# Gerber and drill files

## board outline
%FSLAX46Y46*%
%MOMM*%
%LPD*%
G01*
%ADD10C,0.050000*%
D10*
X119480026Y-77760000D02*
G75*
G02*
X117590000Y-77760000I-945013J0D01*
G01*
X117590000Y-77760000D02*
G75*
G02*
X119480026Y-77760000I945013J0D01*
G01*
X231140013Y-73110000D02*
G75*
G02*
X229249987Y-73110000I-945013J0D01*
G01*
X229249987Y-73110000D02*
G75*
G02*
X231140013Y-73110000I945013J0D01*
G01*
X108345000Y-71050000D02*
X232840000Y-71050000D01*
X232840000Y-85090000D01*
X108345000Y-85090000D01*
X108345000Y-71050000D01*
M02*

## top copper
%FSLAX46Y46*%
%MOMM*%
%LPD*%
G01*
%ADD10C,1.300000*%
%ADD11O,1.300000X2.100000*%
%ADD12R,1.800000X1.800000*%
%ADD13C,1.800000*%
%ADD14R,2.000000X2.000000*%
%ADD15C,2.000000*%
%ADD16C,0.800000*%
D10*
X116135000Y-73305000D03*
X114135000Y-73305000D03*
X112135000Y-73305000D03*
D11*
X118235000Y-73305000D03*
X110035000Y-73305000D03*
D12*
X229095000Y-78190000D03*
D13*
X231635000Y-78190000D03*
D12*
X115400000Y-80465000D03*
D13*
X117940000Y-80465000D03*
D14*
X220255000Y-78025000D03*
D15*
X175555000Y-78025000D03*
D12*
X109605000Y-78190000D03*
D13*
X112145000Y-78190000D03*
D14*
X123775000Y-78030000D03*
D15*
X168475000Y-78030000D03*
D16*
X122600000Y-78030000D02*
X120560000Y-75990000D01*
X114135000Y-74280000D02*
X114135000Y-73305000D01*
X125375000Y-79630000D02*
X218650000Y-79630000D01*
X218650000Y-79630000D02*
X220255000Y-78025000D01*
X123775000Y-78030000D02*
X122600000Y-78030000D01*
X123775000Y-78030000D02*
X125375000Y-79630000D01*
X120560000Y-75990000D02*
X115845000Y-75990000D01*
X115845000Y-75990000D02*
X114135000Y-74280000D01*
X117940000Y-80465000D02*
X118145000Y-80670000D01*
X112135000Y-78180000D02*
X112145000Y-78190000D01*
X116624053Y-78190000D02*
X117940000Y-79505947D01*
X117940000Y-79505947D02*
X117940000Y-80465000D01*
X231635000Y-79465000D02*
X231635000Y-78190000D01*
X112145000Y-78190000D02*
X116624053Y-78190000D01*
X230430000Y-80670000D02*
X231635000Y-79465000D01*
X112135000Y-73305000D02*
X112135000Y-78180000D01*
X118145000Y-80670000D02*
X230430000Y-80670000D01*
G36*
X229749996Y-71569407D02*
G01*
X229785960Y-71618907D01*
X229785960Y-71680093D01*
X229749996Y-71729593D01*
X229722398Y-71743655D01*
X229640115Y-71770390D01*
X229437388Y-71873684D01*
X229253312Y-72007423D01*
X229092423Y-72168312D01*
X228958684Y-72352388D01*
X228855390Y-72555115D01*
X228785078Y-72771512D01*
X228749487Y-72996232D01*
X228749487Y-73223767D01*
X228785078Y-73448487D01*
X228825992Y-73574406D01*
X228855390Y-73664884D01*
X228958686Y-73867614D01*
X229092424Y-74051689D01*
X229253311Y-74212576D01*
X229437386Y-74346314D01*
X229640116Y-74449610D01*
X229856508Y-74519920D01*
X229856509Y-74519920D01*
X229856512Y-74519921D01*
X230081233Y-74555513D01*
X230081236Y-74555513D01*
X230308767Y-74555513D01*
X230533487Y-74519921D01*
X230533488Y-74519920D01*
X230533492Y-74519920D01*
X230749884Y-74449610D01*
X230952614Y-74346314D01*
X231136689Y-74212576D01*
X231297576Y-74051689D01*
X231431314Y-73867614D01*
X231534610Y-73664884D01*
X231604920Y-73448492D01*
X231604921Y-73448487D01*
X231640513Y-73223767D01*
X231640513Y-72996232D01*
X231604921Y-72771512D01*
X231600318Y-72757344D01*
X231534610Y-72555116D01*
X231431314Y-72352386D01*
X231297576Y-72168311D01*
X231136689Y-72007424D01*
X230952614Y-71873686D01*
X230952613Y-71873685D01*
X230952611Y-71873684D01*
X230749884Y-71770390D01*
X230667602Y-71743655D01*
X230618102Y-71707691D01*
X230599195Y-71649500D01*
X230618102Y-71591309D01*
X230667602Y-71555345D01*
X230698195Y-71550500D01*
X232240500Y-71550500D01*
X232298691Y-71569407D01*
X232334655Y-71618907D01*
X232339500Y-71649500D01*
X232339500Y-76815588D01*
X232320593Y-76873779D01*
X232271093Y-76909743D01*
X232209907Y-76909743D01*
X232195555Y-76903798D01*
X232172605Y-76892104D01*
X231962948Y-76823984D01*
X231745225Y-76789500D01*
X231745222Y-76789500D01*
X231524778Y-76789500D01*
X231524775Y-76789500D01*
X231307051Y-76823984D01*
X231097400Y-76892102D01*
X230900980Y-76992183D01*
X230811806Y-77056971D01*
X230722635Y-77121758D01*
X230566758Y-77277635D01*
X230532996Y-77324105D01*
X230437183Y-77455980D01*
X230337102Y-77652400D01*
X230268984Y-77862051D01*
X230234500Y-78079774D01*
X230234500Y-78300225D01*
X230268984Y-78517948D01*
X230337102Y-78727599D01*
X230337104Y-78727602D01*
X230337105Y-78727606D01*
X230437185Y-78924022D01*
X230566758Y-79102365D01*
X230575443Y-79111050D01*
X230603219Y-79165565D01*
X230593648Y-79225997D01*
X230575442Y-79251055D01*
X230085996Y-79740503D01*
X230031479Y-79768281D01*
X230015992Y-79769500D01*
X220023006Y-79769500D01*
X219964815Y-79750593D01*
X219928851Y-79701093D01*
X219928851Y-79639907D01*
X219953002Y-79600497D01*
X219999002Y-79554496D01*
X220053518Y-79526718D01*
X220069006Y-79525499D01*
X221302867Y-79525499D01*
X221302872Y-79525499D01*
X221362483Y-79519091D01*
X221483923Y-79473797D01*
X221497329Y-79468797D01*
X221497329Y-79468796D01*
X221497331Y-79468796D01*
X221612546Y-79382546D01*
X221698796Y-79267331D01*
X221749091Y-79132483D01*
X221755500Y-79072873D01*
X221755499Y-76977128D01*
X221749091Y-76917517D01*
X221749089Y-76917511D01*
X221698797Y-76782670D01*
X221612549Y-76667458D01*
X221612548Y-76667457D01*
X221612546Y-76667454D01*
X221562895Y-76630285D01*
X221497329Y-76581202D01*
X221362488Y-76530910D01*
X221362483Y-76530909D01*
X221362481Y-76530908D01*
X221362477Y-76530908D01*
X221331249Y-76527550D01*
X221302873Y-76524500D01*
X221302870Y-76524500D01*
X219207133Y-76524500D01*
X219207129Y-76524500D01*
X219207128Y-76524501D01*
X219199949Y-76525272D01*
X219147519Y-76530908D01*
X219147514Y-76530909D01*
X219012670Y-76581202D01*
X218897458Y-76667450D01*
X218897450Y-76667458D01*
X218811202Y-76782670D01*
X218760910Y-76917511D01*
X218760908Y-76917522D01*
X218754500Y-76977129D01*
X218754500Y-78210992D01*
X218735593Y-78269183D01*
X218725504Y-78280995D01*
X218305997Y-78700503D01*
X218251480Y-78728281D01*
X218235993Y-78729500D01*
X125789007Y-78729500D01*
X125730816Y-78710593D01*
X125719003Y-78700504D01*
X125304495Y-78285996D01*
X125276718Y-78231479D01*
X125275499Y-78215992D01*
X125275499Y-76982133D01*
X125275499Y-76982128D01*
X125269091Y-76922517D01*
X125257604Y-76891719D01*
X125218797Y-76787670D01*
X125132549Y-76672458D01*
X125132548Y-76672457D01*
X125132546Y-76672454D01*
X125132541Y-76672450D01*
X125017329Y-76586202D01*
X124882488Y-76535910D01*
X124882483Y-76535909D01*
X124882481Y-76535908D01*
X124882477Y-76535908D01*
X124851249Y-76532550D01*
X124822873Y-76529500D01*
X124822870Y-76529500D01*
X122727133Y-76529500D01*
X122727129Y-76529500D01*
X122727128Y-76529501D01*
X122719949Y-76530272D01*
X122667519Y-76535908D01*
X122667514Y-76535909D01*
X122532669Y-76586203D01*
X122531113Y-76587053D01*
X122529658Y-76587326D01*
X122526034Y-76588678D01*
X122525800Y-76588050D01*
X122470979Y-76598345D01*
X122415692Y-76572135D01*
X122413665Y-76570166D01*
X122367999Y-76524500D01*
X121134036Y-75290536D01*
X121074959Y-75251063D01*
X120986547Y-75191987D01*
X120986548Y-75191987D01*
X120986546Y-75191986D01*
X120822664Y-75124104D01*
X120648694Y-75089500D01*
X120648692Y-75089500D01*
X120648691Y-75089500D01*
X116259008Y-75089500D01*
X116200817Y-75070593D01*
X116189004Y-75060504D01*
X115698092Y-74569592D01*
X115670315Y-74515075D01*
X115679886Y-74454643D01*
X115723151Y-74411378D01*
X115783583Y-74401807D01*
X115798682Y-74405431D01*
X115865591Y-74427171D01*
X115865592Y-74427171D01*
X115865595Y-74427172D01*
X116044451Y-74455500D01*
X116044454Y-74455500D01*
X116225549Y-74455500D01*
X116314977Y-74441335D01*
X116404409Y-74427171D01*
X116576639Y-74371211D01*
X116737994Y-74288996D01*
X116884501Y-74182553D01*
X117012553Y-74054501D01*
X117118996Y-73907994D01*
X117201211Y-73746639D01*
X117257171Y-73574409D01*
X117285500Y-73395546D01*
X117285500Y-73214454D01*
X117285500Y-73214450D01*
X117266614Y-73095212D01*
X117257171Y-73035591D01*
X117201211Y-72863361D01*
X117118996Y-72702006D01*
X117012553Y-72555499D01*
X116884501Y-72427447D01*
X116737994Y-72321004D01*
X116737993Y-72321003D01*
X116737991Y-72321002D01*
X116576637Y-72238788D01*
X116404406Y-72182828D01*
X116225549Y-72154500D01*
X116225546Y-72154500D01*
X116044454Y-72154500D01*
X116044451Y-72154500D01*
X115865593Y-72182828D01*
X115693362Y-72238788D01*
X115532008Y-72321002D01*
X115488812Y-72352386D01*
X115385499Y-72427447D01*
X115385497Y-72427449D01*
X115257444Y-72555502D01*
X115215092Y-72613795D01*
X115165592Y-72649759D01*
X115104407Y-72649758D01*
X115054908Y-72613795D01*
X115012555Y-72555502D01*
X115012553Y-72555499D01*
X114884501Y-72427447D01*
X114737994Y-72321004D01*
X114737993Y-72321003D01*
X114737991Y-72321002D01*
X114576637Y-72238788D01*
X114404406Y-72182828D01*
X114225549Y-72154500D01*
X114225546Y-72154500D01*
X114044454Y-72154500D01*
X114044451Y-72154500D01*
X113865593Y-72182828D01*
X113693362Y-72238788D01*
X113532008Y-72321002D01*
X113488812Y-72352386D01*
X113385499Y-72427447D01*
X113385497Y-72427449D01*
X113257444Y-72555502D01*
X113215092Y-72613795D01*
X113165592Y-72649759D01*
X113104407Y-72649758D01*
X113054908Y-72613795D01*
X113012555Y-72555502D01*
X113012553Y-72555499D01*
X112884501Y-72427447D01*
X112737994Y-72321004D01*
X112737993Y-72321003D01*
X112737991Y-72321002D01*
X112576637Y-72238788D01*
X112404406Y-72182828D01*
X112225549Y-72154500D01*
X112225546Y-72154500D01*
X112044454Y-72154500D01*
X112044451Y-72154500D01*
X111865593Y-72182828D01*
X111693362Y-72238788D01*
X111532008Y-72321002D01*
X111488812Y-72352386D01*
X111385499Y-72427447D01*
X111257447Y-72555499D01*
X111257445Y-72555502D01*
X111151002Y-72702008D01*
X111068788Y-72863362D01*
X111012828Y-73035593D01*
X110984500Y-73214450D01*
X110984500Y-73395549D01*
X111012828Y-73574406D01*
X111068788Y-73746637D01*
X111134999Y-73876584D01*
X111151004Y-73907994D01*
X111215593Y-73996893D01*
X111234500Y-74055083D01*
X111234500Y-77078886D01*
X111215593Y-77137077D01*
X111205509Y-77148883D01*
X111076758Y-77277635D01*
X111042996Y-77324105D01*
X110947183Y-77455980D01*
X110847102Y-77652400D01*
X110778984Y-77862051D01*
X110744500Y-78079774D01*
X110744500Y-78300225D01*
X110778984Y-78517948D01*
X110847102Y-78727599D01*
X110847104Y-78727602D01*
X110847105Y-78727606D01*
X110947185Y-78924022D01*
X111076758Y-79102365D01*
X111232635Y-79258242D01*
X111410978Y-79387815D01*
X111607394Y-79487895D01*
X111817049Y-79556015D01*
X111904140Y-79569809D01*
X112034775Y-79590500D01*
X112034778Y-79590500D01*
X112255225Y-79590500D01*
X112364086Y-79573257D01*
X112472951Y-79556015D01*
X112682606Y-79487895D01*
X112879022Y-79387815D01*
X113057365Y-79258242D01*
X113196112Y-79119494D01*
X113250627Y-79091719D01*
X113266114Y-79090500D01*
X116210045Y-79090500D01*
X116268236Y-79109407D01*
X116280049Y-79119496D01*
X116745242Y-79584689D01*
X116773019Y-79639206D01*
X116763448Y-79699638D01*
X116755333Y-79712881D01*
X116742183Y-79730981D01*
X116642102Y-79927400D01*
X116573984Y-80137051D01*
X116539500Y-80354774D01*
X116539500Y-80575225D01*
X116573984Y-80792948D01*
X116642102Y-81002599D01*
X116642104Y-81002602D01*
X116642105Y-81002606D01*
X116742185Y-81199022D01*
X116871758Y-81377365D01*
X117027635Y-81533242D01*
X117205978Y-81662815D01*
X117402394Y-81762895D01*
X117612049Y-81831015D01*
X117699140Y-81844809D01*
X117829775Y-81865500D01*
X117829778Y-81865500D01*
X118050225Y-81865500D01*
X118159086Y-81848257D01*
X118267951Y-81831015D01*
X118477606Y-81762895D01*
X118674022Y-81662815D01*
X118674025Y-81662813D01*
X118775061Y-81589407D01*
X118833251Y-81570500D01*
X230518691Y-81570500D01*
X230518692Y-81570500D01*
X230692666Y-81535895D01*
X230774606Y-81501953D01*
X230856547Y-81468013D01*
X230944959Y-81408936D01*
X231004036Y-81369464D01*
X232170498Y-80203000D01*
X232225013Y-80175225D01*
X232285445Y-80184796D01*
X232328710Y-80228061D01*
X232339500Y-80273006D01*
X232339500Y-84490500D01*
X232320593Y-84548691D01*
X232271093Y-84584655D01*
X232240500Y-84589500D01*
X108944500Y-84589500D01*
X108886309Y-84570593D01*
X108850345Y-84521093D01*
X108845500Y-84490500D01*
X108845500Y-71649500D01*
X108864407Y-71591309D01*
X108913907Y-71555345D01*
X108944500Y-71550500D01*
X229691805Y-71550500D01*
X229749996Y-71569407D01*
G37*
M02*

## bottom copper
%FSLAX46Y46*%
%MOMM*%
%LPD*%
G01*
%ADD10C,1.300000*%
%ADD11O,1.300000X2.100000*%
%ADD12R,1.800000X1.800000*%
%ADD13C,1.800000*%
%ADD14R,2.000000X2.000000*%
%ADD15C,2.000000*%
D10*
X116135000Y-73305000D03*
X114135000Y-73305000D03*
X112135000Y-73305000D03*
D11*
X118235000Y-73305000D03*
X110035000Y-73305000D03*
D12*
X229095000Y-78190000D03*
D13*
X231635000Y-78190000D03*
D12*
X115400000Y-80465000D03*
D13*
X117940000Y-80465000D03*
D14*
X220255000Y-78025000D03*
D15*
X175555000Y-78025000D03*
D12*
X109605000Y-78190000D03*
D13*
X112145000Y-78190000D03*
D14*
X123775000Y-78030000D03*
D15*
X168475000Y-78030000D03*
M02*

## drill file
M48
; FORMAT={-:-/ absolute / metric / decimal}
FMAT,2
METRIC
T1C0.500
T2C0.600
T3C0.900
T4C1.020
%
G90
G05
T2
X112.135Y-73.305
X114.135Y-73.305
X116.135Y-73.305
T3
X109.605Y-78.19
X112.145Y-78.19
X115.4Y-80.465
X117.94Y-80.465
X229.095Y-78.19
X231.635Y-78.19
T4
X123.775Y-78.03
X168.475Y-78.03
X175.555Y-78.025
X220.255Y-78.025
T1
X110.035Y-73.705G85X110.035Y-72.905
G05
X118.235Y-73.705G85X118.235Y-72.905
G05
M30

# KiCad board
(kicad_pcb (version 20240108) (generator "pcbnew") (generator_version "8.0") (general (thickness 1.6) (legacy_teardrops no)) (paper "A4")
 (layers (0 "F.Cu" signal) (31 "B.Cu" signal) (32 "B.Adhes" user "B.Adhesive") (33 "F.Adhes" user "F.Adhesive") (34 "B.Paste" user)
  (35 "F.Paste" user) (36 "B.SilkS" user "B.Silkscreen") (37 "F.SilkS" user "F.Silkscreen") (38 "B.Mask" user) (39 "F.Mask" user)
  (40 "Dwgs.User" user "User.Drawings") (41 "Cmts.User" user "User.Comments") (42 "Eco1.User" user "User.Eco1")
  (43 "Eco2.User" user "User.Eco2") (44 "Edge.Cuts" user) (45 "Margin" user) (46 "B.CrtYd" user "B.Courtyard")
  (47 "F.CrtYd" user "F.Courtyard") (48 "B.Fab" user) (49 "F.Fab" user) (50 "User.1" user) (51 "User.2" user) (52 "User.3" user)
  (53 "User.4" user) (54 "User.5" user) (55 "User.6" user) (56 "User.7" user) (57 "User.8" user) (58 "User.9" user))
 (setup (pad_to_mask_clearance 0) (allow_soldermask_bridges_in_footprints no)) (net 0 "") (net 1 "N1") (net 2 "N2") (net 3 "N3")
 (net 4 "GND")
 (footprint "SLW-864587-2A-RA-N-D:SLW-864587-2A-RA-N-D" (layer "F.Cu") (at 114.135 73.305 180)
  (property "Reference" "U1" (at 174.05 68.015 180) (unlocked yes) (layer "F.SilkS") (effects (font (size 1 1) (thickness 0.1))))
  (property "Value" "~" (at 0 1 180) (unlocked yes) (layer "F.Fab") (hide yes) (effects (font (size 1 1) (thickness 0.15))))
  (pad "1" thru_hole circle (at -2 0 180) (size 1.3 1.3) (drill 0.6) (layers "*.Cu" "*.Mask") (remove_unused_layers no) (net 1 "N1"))
  (pad "2" thru_hole circle (at 0 0 180) (size 1.3 1.3) (drill 0.6) (layers "*.Cu" "*.Mask") (remove_unused_layers no) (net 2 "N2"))
  (pad "3" thru_hole circle (at 2 0 180) (size 1.3 1.3) (drill 0.6) (layers "*.Cu" "*.Mask") (remove_unused_layers no) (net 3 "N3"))
  (pad "4" thru_hole oval (at -4.1 0 180) (size 1.3 2.1) (drill oval 0.5 1.3) (layers "*.Cu" "*.Mask") (remove_unused_layers no)
   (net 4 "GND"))
  (pad "5" thru_hole oval (at 4.1 0 180) (size 1.3 2.1) (drill oval 0.5 1.3) (layers "*.Cu" "*.Mask") (remove_unused_layers no)
   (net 4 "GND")))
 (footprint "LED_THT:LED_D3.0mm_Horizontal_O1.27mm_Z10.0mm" (layer "F.Cu") (at 229.095 78.19)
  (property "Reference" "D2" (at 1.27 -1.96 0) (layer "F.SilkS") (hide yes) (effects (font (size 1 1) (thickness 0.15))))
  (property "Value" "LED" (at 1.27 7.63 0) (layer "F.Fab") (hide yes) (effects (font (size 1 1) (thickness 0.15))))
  (pad "1" thru_hole rect (at 0 0) (size 1.8 1.8) (drill 0.9) (layers "*.Cu" "*.Mask") (remove_unused_layers no) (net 4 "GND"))
  (pad "2" thru_hole circle (at 2.54 0) (size 1.8 1.8) (drill 0.9) (layers "*.Cu" "*.Mask") (remove_unused_layers no) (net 3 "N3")))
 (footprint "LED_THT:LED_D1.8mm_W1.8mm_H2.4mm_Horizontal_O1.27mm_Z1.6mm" (layer "F.Cu") (at 115.4 80.465)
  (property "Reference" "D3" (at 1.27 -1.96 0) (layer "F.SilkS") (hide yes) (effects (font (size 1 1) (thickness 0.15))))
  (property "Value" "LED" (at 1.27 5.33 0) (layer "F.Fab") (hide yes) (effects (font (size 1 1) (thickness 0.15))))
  (pad "1" thru_hole rect (at 0 0) (size 1.8 1.8) (drill 0.9) (layers "*.Cu" "*.Mask") (remove_unused_layers no) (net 4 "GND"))
  (pad "2" thru_hole circle (at 2.54 0) (size 1.8 1.8) (drill 0.9) (layers "*.Cu" "*.Mask") (remove_unused_layers no) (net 3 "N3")))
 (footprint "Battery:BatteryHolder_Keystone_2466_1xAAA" (layer "F.Cu") (at 220.255 78.025 180)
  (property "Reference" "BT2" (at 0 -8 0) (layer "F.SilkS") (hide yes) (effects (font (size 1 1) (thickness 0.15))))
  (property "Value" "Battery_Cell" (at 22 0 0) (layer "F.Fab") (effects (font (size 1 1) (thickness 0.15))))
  (pad "1" thru_hole rect (at 0 0 180) (size 2 2) (drill 1.02) (layers "*.Cu" "*.Mask") (remove_unused_layers no) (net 2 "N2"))
  (pad "2" thru_hole circle (at 44.7 0 180) (size 2 2) (drill 1.02) (layers "*.Cu" "*.Mask") (remove_unused_layers no) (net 4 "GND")))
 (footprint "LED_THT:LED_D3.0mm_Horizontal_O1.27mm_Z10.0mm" (layer "F.Cu") (at 109.605 78.19)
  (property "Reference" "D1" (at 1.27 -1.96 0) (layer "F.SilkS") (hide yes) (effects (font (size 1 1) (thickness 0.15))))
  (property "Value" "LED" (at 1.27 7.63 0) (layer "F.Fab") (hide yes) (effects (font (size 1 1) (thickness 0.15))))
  (pad "1" thru_hole rect (at 0 0) (size 1.8 1.8) (drill 0.9) (layers "*.Cu" "*.Mask") (remove_unused_layers no) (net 4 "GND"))
  (pad "2" thru_hole circle (at 2.54 0) (size 1.8 1.8) (drill 0.9) (layers "*.Cu" "*.Mask") (remove_unused_layers no) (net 3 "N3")))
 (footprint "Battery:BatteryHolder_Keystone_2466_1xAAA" (layer "F.Cu") (at 123.775 78.03)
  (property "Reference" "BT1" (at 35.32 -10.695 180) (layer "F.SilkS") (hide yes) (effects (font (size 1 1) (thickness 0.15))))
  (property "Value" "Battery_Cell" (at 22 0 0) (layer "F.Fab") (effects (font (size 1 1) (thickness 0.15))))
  (pad "1" thru_hole rect (at 0 0) (size 2 2) (drill 1.02) (layers "*.Cu" "*.Mask") (remove_unused_layers no) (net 2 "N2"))
  (pad "2" thru_hole circle (at 44.7 0) (size 2 2) (drill 1.02) (layers "*.Cu" "*.Mask") (remove_unused_layers no) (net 4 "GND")))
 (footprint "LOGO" (layer "B.Cu") (at 197.90575 77.885181 180)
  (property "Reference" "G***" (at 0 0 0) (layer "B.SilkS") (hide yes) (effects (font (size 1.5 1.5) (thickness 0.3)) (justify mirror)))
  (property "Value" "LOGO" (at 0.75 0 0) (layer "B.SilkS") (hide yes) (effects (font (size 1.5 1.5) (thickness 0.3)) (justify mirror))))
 (gr_circle (center 118.535013 77.76) (end 119.480013 77.755) (stroke (width 0.05) (type default)) (fill none) (layer "Edge.Cuts"))
 (gr_circle (center 230.195 73.11) (end 231.14 73.105) (stroke (width 0.05) (type default)) (fill none) (layer "Edge.Cuts"))
 (gr_rect (start 108.345 71.05) (end 232.84 85.09) (stroke (width 0.05) (type default)) (fill none) (layer "Edge.Cuts"))
 (segment (start 122.6 78.03) (end 120.56 75.99) (width 0.8) (layer "F.Cu") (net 2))
 (segment (start 114.135 74.28) (end 114.135 73.305) (width 0.8) (layer "F.Cu") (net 2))
 (segment (start 125.375 79.63) (end 218.65 79.63) (width 0.8) (layer "F.Cu") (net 2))
 (segment (start 218.65 79.63) (end 220.255 78.025) (width 0.8) (layer "F.Cu") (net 2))
 (segment (start 123.775 78.03) (end 122.6 78.03) (width 0.8) (layer "F.Cu") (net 2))
 (segment (start 123.775 78.03) (end 125.375 79.63) (width 0.8) (layer "F.Cu") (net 2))
 (segment (start 120.56 75.99) (end 115.845 75.99) (width 0.8) (layer "F.Cu") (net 2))
 (segment (start 115.845 75.99) (end 114.135 74.28) (width 0.8) (layer "F.Cu") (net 2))
 (segment (start 117.94 80.465) (end 118.145 80.67) (width 0.8) (layer "F.Cu") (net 3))
 (segment (start 112.135 78.18) (end 112.145 78.19) (width 0.8) (layer "F.Cu") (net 3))
 (segment (start 116.624053 78.19) (end 117.94 79.505947) (width 0.8) (layer "F.Cu") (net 3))
 (segment (start 117.94 79.505947) (end 117.94 80.465) (width 0.8) (layer "F.Cu") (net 3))
 (segment (start 231.635 79.465) (end 231.635 78.19) (width 0.8) (layer "F.Cu") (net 3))
 (segment (start 112.145 78.19) (end 116.624053 78.19) (width 0.8) (layer "F.Cu") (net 3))
 (segment (start 230.43 80.67) (end 231.635 79.465) (width 0.8) (layer "F.Cu") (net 3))
 (segment (start 112.135 73.305) (end 112.135 78.18) (width 0.8) (layer "F.Cu") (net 3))
 (segment (start 118.145 80.67) (end 230.43 80.67) (width 0.8) (layer "F.Cu") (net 3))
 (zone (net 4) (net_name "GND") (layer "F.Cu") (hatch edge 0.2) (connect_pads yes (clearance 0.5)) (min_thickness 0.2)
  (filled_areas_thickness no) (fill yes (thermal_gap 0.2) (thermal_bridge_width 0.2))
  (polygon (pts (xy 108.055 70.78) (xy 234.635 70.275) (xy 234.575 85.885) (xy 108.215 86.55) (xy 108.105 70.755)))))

